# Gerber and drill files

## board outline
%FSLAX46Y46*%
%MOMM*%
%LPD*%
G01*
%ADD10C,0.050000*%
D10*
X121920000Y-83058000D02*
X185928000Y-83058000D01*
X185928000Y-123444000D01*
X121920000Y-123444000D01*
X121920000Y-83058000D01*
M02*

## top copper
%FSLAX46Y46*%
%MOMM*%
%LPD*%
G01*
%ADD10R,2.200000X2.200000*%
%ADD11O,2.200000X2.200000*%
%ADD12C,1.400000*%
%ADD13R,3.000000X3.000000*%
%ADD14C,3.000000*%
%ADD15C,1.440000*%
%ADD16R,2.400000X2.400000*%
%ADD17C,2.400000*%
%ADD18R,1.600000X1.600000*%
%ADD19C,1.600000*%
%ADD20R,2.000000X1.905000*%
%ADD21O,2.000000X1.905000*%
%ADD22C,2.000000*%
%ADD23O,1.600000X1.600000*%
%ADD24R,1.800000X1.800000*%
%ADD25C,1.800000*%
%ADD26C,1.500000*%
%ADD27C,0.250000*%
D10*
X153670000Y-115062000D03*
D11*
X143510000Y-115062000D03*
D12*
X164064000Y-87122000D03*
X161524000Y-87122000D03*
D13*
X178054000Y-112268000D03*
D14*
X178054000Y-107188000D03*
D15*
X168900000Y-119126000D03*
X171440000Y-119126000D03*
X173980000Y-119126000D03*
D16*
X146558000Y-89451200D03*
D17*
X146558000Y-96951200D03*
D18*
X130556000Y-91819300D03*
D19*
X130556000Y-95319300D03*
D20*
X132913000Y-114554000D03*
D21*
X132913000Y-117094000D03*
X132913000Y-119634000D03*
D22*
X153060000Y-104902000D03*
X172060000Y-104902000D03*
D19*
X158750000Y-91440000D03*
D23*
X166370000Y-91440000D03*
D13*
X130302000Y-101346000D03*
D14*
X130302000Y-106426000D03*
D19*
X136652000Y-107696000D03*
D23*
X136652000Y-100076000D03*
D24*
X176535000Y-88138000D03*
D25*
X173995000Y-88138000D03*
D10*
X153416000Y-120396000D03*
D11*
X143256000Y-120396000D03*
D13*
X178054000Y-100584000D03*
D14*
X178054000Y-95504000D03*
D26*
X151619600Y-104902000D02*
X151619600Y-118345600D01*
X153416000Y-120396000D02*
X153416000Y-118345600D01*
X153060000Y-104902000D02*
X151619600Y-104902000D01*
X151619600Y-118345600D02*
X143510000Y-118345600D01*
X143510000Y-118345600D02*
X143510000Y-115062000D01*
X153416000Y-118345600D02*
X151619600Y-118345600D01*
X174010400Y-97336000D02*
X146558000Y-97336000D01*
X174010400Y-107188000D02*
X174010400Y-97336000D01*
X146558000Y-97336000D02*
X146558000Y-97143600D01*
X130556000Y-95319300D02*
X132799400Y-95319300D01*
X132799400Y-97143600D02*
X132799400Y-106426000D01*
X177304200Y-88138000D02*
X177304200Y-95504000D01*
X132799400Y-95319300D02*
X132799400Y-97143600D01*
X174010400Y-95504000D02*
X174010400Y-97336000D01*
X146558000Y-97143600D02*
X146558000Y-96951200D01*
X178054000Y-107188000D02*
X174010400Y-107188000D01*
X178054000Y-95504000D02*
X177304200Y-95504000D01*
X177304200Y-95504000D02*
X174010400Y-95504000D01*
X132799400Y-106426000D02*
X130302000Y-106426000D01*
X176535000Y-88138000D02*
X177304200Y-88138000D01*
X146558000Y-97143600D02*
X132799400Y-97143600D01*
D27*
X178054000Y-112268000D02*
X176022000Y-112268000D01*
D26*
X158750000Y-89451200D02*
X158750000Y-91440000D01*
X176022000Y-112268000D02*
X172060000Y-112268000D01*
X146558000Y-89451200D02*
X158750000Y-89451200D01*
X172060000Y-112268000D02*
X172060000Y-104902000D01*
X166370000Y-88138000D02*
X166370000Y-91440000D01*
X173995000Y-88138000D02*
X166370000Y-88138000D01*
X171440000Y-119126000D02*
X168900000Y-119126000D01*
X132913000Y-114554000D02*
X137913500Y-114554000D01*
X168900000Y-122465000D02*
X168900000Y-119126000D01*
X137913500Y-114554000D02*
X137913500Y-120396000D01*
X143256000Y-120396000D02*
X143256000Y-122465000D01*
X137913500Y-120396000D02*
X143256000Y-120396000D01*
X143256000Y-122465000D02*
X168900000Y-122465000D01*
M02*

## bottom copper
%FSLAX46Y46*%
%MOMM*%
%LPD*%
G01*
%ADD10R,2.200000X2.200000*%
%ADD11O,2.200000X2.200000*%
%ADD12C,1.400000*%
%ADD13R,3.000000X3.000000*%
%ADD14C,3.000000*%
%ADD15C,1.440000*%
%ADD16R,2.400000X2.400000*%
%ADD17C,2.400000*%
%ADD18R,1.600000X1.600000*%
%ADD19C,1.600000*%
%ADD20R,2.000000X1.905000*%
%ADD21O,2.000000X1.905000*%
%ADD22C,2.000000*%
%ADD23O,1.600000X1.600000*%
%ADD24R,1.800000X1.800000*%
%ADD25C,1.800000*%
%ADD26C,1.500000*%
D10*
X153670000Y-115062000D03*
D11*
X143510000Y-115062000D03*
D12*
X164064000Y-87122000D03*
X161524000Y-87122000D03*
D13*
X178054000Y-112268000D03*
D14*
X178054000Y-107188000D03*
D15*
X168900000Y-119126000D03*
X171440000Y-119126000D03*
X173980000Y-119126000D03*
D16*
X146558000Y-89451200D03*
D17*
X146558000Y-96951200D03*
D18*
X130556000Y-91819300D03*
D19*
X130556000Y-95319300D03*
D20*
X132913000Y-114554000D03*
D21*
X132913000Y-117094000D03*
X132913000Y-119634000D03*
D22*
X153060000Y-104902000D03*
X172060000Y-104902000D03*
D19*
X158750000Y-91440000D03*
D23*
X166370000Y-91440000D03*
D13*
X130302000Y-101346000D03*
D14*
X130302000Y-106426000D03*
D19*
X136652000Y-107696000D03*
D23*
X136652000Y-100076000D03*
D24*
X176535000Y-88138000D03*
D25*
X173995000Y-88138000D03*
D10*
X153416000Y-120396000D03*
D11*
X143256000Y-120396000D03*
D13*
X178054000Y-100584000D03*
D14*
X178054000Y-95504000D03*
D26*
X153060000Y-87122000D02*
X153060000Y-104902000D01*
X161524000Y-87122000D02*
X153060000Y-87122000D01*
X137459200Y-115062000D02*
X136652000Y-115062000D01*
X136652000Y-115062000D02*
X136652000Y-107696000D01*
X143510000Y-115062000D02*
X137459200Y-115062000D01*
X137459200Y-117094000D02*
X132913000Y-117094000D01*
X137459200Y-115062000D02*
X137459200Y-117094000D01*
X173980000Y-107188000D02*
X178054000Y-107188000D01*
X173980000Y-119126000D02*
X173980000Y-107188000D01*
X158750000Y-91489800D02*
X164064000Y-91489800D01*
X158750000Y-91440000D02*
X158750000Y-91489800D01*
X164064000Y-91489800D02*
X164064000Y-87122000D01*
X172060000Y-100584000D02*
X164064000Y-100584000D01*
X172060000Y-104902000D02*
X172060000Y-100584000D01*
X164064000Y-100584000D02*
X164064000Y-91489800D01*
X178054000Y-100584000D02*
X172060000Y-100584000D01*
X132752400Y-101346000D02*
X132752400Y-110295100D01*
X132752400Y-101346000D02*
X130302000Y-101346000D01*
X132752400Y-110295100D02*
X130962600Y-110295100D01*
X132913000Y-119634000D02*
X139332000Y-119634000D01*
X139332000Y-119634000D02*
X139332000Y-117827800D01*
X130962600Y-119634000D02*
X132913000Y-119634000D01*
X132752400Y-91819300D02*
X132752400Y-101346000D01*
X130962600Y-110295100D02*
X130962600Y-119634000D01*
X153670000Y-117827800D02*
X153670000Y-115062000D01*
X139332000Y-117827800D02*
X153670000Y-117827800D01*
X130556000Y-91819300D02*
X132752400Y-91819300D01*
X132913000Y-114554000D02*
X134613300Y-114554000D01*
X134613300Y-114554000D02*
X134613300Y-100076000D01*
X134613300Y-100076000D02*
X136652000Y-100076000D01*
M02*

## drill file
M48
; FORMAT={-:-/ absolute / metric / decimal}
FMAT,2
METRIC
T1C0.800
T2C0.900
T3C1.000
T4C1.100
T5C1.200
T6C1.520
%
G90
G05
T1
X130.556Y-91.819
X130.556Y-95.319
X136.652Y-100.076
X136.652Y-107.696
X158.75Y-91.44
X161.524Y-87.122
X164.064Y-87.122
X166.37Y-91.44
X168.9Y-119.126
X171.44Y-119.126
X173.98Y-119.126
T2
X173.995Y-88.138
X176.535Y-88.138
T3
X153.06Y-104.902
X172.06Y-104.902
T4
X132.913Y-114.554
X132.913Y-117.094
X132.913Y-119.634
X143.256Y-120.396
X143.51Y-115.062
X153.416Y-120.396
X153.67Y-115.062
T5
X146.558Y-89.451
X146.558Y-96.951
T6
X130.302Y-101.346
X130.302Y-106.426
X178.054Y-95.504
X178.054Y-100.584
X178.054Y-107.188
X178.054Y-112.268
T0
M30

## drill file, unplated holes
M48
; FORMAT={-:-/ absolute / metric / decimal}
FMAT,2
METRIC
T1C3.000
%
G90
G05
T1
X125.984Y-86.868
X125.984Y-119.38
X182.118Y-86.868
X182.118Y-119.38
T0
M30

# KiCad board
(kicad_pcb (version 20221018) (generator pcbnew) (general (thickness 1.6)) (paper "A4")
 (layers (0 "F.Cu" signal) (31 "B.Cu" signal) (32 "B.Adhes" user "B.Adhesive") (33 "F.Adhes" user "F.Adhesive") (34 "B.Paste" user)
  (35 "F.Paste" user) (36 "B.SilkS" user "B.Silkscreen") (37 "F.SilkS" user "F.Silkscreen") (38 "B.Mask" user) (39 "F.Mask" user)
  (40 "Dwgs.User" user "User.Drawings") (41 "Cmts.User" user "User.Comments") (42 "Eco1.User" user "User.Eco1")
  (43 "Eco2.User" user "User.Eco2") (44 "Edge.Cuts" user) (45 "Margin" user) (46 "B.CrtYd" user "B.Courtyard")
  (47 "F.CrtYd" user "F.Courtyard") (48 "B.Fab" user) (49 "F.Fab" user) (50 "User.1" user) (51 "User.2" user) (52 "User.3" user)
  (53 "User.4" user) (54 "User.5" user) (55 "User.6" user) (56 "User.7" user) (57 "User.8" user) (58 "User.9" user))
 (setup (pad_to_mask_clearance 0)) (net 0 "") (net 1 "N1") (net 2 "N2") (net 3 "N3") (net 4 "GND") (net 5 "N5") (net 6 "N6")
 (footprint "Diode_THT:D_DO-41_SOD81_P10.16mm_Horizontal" (layer "F.Cu") (at 153.67 115.062 180)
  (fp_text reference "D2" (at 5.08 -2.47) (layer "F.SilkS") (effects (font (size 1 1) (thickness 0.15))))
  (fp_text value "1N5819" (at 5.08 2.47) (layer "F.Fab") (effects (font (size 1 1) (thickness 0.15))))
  (pad "1" thru_hole rect (at 0 0 180) (size 2.2 2.2) (drill 1.1) (layers "*.Cu" "*.Mask") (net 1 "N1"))
  (pad "2" thru_hole oval (at 10.16 0 180) (size 2.2 2.2) (drill 1.1) (layers "*.Cu" "*.Mask") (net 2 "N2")))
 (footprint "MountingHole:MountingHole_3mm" (layer "F.Cu") (at 125.984 86.868)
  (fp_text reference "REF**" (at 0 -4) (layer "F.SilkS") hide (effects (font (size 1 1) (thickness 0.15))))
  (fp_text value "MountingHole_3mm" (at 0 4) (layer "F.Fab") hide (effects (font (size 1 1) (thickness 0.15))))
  (pad "" np_thru_hole circle (at 0 0) (size 3 3) (drill 3) (layers "*.Cu" "*.Mask")))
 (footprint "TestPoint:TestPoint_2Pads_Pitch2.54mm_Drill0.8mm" (layer "F.Cu") (at 164.064 87.122 180)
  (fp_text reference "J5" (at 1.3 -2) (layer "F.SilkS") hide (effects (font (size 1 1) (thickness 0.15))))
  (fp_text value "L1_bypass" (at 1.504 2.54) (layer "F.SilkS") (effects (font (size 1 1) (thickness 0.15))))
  (pad "1" thru_hole circle (at 0 0 180) (size 1.4 1.4) (drill 0.8) (layers "*.Cu" "*.Mask") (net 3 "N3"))
  (pad "2" thru_hole circle (at 2.54 0 180) (size 1.4 1.4) (drill 0.8) (layers "*.Cu" "*.Mask") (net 2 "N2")))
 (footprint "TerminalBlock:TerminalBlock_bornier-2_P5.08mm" (layer "F.Cu") (at 178.054 112.268 90)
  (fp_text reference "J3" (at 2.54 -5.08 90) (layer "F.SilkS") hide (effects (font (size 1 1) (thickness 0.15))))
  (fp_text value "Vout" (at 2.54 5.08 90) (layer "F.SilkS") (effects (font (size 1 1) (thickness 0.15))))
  (pad "1" thru_hole rect (at 0 0 90) (size 3 3) (drill 1.52) (layers "*.Cu" "*.Mask") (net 3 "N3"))
  (pad "2" thru_hole circle (at 5.08 0 90) (size 3 3) (drill 1.52) (layers "*.Cu" "*.Mask") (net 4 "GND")))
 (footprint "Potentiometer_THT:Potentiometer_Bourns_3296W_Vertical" (layer "F.Cu") (at 168.9 119.126 180)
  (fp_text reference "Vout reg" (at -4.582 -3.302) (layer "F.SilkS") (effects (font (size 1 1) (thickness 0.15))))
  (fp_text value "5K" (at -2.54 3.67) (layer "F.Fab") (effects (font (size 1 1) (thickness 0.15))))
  (pad "1" thru_hole circle (at 0 0 180) (size 1.44 1.44) (drill 0.8) (layers "*.Cu" "*.Mask") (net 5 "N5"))
  (pad "2" thru_hole circle (at -2.54 0 180) (size 1.44 1.44) (drill 0.8) (layers "*.Cu" "*.Mask") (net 5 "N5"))
  (pad "3" thru_hole circle (at -5.08 0 180) (size 1.44 1.44) (drill 0.8) (layers "*.Cu" "*.Mask") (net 4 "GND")))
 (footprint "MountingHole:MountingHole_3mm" (layer "F.Cu") (at 182.118 86.868)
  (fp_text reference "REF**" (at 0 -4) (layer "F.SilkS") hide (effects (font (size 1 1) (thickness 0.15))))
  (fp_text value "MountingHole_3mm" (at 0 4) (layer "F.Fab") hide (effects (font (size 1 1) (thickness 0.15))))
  (pad "" np_thru_hole circle (at 0 0) (size 3 3) (drill 3) (layers "*.Cu" "*.Mask")))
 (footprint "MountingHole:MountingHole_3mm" (layer "F.Cu") (at 125.984 119.38)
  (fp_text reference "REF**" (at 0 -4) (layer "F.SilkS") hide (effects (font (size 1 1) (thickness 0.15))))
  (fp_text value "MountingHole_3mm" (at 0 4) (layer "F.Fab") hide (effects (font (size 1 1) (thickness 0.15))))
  (pad "" np_thru_hole circle (at 0 0) (size 3 3) (drill 3) (layers "*.Cu" "*.Mask")))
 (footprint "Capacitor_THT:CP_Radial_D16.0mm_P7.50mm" (layer "F.Cu") (at 146.558 89.4512 -90)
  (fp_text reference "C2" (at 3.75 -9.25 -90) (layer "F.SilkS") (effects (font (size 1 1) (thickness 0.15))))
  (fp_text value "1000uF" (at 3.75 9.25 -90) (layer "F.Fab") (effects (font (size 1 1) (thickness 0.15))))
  (pad "1" thru_hole rect (at 0 0 270) (size 2.4 2.4) (drill 1.2) (layers "*.Cu" "*.Mask") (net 3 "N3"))
  (pad "2" thru_hole circle (at 7.5 0 270) (size 2.4 2.4) (drill 1.2) (layers "*.Cu" "*.Mask") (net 4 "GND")))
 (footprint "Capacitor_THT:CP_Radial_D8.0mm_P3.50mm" (layer "F.Cu") (at 130.556 91.8193 -90)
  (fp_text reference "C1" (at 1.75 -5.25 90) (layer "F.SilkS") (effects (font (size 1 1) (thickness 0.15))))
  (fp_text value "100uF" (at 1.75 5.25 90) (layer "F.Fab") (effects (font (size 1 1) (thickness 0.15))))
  (pad "1" thru_hole rect (at 0 0 270) (size 1.6 1.6) (drill 0.8) (layers "*.Cu" "*.Mask") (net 1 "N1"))
  (pad "2" thru_hole circle (at 3.5 0 270) (size 1.6 1.6) (drill 0.8) (layers "*.Cu" "*.Mask") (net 4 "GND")))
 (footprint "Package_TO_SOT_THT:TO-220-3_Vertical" (layer "F.Cu") (at 132.913 114.554 -90)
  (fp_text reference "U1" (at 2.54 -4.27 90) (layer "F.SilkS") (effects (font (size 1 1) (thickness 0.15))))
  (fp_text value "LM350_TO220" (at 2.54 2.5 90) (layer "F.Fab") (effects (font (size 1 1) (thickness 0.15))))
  (pad "1" thru_hole rect (at 0 0 270) (size 1.905 2) (drill 1.1) (layers "*.Cu" "*.Mask") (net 5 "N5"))
  (pad "2" thru_hole oval (at 2.54 0 270) (size 1.905 2) (drill 1.1) (layers "*.Cu" "*.Mask") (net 2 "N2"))
  (pad "3" thru_hole oval (at 5.08 0 270) (size 1.905 2) (drill 1.1) (layers "*.Cu" "*.Mask") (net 1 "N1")))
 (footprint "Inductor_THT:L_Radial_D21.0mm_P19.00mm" (layer "F.Cu") (at 153.06 104.902)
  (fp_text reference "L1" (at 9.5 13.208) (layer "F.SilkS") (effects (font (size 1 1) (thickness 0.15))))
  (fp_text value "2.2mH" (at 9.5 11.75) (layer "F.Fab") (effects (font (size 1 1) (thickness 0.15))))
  (pad "1" thru_hole circle (at 0 0) (size 2 2) (drill 1) (layers "*.Cu" "*.Mask") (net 2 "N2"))
  (pad "2" thru_hole circle (at 19 0) (size 2 2) (drill 1) (layers "*.Cu" "*.Mask") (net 3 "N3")))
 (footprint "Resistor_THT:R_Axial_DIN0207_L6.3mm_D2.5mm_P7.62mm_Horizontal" (layer "F.Cu") (at 158.75 91.44)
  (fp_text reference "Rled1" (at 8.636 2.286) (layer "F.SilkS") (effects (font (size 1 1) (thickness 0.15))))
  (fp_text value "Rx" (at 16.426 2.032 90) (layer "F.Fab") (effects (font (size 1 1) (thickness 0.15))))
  (pad "1" thru_hole circle (at 0 0) (size 1.6 1.6) (drill 0.8) (layers "*.Cu" "*.Mask") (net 3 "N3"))
  (pad "2" thru_hole oval (at 7.62 0) (size 1.6 1.6) (drill 0.8) (layers "*.Cu" "*.Mask") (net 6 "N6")))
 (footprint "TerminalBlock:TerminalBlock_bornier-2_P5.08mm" (layer "F.Cu") (at 130.302 101.346 -90)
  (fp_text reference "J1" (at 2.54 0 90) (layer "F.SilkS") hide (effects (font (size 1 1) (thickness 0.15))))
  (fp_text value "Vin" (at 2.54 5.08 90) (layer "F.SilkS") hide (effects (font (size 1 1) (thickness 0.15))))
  (pad "1" thru_hole rect (at 0 0 270) (size 3 3) (drill 1.52) (layers "*.Cu" "*.Mask") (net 1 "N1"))
  (pad "2" thru_hole circle (at 5.08 0 270) (size 3 3) (drill 1.52) (layers "*.Cu" "*.Mask") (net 4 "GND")))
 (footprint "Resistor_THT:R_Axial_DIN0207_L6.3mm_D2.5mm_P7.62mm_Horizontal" (layer "F.Cu") (at 136.652 107.696 90)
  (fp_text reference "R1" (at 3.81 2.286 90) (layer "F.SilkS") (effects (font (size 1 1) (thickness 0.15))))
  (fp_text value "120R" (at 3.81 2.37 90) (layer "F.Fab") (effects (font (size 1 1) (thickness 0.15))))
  (pad "1" thru_hole circle (at 0 0 90) (size 1.6 1.6) (drill 0.8) (layers "*.Cu" "*.Mask") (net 2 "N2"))
  (pad "2" thru_hole oval (at 7.62 0 90) (size 1.6 1.6) (drill 0.8) (layers "*.Cu" "*.Mask") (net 5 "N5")))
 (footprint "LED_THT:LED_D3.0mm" (layer "F.Cu") (at 176.535 88.138 180)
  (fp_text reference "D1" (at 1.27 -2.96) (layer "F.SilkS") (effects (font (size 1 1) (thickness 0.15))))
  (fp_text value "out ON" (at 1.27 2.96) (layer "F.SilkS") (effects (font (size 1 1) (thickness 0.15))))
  (pad "1" thru_hole rect (at 0 0 180) (size 1.8 1.8) (drill 0.9) (layers "*.Cu" "*.Mask") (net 4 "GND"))
  (pad "2" thru_hole circle (at 2.54 0 180) (size 1.8 1.8) (drill 0.9) (layers "*.Cu" "*.Mask") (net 6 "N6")))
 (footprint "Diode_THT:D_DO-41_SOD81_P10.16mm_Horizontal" (layer "F.Cu") (at 153.416 120.396 180)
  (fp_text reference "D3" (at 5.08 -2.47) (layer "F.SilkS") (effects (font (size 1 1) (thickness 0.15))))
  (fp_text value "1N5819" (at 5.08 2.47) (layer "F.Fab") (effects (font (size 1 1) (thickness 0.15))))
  (pad "1" thru_hole rect (at 0 0 180) (size 2.2 2.2) (drill 1.1) (layers "*.Cu" "*.Mask") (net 2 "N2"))
  (pad "2" thru_hole oval (at 10.16 0 180) (size 2.2 2.2) (drill 1.1) (layers "*.Cu" "*.Mask") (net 5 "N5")))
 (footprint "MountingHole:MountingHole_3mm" (layer "F.Cu") (at 182.118 119.38)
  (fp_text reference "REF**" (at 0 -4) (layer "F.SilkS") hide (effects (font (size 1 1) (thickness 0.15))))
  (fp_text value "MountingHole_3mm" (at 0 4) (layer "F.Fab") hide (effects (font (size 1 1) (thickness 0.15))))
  (pad "" np_thru_hole circle (at 0 0) (size 3 3) (drill 3) (layers "*.Cu" "*.Mask")))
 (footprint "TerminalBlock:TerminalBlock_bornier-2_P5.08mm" (layer "F.Cu") (at 178.054 100.584 90)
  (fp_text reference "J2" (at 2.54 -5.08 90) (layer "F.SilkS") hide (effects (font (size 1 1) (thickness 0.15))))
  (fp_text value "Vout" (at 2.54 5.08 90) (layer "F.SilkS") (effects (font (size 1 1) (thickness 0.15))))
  (pad "1" thru_hole rect (at 0 0 90) (size 3 3) (drill 1.52) (layers "*.Cu" "*.Mask") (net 3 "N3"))
  (pad "2" thru_hole circle (at 5.08 0 90) (size 3 3) (drill 1.52) (layers "*.Cu" "*.Mask") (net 4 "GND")))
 (gr_rect (start 121.92 83.058) (end 185.928 123.444) (stroke (width 0.05) (type solid)) (fill none) (layer "Edge.Cuts"))
 (segment (start 151.6196 104.902) (end 151.6196 118.3456) (width 1.5) (layer "F.Cu") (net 2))
 (segment (start 153.416 120.396) (end 153.416 118.3456) (width 1.5) (layer "F.Cu") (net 2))
 (segment (start 153.06 104.902) (end 151.6196 104.902) (width 1.5) (layer "F.Cu") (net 2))
 (segment (start 151.6196 118.3456) (end 143.51 118.3456) (width 1.5) (layer "F.Cu") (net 2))
 (segment (start 143.51 118.3456) (end 143.51 115.062) (width 1.5) (layer "F.Cu") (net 2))
 (segment (start 153.416 118.3456) (end 151.6196 118.3456) (width 1.5) (layer "F.Cu") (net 2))
 (segment (start 153.06 87.122) (end 153.06 104.902) (width 1.5) (layer "B.Cu") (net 2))
 (segment (start 161.524 87.122) (end 153.06 87.122) (width 1.5) (layer "B.Cu") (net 2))
 (segment (start 137.4592 115.062) (end 136.652 115.062) (width 1.5) (layer "B.Cu") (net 2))
 (segment (start 136.652 115.062) (end 136.652 107.696) (width 1.5) (layer "B.Cu") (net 2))
 (segment (start 143.51 115.062) (end 137.4592 115.062) (width 1.5) (layer "B.Cu") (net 2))
 (segment (start 137.4592 117.094) (end 132.913 117.094) (width 1.5) (layer "B.Cu") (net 2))
 (segment (start 137.4592 115.062) (end 137.4592 117.094) (width 1.5) (layer "B.Cu") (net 2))
 (segment (start 174.0104 97.336) (end 146.558 97.336) (width 1.5) (layer "F.Cu") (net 4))
 (segment (start 174.0104 107.188) (end 174.0104 97.336) (width 1.5) (layer "F.Cu") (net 4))
 (segment (start 146.558 97.336) (end 146.558 97.1436) (width 1.5) (layer "F.Cu") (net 4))
 (segment (start 130.556 95.3193) (end 132.7994 95.3193) (width 1.5) (layer "F.Cu") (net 4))
 (segment (start 132.7994 97.1436) (end 132.7994 106.426) (width 1.5) (layer "F.Cu") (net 4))
 (segment (start 177.3042 88.138) (end 177.3042 95.504) (width 1.5) (layer "F.Cu") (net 4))
 (segment (start 132.7994 95.3193) (end 132.7994 97.1436) (width 1.5) (layer "F.Cu") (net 4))
 (segment (start 174.0104 95.504) (end 174.0104 97.336) (width 1.5) (layer "F.Cu") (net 4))
 (segment (start 146.558 97.1436) (end 146.558 96.9512) (width 1.5) (layer "F.Cu") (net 4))
 (segment (start 178.054 107.188) (end 174.0104 107.188) (width 1.5) (layer "F.Cu") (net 4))
 (segment (start 178.054 95.504) (end 177.3042 95.504) (width 1.5) (layer "F.Cu") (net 4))
 (segment (start 177.3042 95.504) (end 174.0104 95.504) (width 1.5) (layer "F.Cu") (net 4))
 (segment (start 132.7994 106.426) (end 130.302 106.426) (width 1.5) (layer "F.Cu") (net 4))
 (segment (start 176.535 88.138) (end 177.3042 88.138) (width 1.5) (layer "F.Cu") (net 4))
 (segment (start 146.558 97.1436) (end 132.7994 97.1436) (width 1.5) (layer "F.Cu") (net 4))
 (segment (start 173.98 107.188) (end 178.054 107.188) (width 1.5) (layer "B.Cu") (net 4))
 (segment (start 173.98 119.126) (end 173.98 107.188) (width 1.5) (layer "B.Cu") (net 4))
 (segment (start 178.054 112.268) (end 176.022 112.268) (width 0.25) (layer "F.Cu") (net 3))
 (segment (start 158.75 89.4512) (end 158.75 91.44) (width 1.5) (layer "F.Cu") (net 3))
 (segment (start 176.022 112.268) (end 172.06 112.268) (width 1.5) (layer "F.Cu") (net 3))
 (segment (start 146.558 89.4512) (end 158.75 89.4512) (width 1.5) (layer "F.Cu") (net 3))
 (segment (start 172.06 112.268) (end 172.06 104.902) (width 1.5) (layer "F.Cu") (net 3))
 (segment (start 158.75 91.4898) (end 164.064 91.4898) (width 1.5) (layer "B.Cu") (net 3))
 (segment (start 158.75 91.44) (end 158.75 91.4898) (width 1.5) (layer "B.Cu") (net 3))
 (segment (start 164.064 91.4898) (end 164.064 87.122) (width 1.5) (layer "B.Cu") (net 3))
 (segment (start 172.06 100.584) (end 164.064 100.584) (width 1.5) (layer "B.Cu") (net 3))
 (segment (start 172.06 104.902) (end 172.06 100.584) (width 1.5) (layer "B.Cu") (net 3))
 (segment (start 164.064 100.584) (end 164.064 91.4898) (width 1.5) (layer "B.Cu") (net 3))
 (segment (start 178.054 100.584) (end 172.06 100.584) (width 1.5) (layer "B.Cu") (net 3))
 (segment (start 166.37 88.138) (end 166.37 91.44) (width 1.5) (layer "F.Cu") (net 6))
 (segment (start 173.995 88.138) (end 166.37 88.138) (width 1.5) (layer "F.Cu") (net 6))
 (segment (start 132.7524 101.346) (end 132.7524 110.2951) (width 1.5) (layer "B.Cu") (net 1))
 (segment (start 132.7524 101.346) (end 130.302 101.346) (width 1.5) (layer "B.Cu") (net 1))
 (segment (start 132.7524 110.2951) (end 130.9626 110.2951) (width 1.5) (layer "B.Cu") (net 1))
 (segment (start 132.913 119.634) (end 139.332 119.634) (width 1.5) (layer "B.Cu") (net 1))
 (segment (start 139.332 119.634) (end 139.332 117.8278) (width 1.5) (layer "B.Cu") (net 1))
 (segment (start 130.9626 119.634) (end 132.913 119.634) (width 1.5) (layer "B.Cu") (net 1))
 (segment (start 132.7524 91.8193) (end 132.7524 101.346) (width 1.5) (layer "B.Cu") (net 1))
 (segment (start 130.9626 110.2951) (end 130.9626 119.634) (width 1.5) (layer "B.Cu") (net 1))
 (segment (start 153.67 117.8278) (end 153.67 115.062) (width 1.5) (layer "B.Cu") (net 1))
 (segment (start 139.332 117.8278) (end 153.67 117.8278) (width 1.5) (layer "B.Cu") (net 1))
 (segment (start 130.556 91.8193) (end 132.7524 91.8193) (width 1.5) (layer "B.Cu") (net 1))
 (segment (start 171.44 119.126) (end 168.9 119.126) (width 1.5) (layer "F.Cu") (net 5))
 (segment (start 132.913 114.554) (end 137.9135 114.554) (width 1.5) (layer "F.Cu") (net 5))
 (segment (start 168.9 122.465) (end 168.9 119.126) (width 1.5) (layer "F.Cu") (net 5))
 (segment (start 137.9135 114.554) (end 137.9135 120.396) (width 1.5) (layer "F.Cu") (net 5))
 (segment (start 143.256 120.396) (end 143.256 122.465) (width 1.5) (layer "F.Cu") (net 5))
 (segment (start 137.9135 120.396) (end 143.256 120.396) (width 1.5) (layer "F.Cu") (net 5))
 (segment (start 143.256 122.465) (end 168.9 122.465) (width 1.5) (layer "F.Cu") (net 5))
 (segment (start 132.913 114.554) (end 134.6133 114.554) (width 1.5) (layer "B.Cu") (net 5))
 (segment (start 134.6133 114.554) (end 134.6133 100.076) (width 1.5) (layer "B.Cu") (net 5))
 (segment (start 134.6133 100.076) (end 136.652 100.076) (width 1.5) (layer "B.Cu") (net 5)))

